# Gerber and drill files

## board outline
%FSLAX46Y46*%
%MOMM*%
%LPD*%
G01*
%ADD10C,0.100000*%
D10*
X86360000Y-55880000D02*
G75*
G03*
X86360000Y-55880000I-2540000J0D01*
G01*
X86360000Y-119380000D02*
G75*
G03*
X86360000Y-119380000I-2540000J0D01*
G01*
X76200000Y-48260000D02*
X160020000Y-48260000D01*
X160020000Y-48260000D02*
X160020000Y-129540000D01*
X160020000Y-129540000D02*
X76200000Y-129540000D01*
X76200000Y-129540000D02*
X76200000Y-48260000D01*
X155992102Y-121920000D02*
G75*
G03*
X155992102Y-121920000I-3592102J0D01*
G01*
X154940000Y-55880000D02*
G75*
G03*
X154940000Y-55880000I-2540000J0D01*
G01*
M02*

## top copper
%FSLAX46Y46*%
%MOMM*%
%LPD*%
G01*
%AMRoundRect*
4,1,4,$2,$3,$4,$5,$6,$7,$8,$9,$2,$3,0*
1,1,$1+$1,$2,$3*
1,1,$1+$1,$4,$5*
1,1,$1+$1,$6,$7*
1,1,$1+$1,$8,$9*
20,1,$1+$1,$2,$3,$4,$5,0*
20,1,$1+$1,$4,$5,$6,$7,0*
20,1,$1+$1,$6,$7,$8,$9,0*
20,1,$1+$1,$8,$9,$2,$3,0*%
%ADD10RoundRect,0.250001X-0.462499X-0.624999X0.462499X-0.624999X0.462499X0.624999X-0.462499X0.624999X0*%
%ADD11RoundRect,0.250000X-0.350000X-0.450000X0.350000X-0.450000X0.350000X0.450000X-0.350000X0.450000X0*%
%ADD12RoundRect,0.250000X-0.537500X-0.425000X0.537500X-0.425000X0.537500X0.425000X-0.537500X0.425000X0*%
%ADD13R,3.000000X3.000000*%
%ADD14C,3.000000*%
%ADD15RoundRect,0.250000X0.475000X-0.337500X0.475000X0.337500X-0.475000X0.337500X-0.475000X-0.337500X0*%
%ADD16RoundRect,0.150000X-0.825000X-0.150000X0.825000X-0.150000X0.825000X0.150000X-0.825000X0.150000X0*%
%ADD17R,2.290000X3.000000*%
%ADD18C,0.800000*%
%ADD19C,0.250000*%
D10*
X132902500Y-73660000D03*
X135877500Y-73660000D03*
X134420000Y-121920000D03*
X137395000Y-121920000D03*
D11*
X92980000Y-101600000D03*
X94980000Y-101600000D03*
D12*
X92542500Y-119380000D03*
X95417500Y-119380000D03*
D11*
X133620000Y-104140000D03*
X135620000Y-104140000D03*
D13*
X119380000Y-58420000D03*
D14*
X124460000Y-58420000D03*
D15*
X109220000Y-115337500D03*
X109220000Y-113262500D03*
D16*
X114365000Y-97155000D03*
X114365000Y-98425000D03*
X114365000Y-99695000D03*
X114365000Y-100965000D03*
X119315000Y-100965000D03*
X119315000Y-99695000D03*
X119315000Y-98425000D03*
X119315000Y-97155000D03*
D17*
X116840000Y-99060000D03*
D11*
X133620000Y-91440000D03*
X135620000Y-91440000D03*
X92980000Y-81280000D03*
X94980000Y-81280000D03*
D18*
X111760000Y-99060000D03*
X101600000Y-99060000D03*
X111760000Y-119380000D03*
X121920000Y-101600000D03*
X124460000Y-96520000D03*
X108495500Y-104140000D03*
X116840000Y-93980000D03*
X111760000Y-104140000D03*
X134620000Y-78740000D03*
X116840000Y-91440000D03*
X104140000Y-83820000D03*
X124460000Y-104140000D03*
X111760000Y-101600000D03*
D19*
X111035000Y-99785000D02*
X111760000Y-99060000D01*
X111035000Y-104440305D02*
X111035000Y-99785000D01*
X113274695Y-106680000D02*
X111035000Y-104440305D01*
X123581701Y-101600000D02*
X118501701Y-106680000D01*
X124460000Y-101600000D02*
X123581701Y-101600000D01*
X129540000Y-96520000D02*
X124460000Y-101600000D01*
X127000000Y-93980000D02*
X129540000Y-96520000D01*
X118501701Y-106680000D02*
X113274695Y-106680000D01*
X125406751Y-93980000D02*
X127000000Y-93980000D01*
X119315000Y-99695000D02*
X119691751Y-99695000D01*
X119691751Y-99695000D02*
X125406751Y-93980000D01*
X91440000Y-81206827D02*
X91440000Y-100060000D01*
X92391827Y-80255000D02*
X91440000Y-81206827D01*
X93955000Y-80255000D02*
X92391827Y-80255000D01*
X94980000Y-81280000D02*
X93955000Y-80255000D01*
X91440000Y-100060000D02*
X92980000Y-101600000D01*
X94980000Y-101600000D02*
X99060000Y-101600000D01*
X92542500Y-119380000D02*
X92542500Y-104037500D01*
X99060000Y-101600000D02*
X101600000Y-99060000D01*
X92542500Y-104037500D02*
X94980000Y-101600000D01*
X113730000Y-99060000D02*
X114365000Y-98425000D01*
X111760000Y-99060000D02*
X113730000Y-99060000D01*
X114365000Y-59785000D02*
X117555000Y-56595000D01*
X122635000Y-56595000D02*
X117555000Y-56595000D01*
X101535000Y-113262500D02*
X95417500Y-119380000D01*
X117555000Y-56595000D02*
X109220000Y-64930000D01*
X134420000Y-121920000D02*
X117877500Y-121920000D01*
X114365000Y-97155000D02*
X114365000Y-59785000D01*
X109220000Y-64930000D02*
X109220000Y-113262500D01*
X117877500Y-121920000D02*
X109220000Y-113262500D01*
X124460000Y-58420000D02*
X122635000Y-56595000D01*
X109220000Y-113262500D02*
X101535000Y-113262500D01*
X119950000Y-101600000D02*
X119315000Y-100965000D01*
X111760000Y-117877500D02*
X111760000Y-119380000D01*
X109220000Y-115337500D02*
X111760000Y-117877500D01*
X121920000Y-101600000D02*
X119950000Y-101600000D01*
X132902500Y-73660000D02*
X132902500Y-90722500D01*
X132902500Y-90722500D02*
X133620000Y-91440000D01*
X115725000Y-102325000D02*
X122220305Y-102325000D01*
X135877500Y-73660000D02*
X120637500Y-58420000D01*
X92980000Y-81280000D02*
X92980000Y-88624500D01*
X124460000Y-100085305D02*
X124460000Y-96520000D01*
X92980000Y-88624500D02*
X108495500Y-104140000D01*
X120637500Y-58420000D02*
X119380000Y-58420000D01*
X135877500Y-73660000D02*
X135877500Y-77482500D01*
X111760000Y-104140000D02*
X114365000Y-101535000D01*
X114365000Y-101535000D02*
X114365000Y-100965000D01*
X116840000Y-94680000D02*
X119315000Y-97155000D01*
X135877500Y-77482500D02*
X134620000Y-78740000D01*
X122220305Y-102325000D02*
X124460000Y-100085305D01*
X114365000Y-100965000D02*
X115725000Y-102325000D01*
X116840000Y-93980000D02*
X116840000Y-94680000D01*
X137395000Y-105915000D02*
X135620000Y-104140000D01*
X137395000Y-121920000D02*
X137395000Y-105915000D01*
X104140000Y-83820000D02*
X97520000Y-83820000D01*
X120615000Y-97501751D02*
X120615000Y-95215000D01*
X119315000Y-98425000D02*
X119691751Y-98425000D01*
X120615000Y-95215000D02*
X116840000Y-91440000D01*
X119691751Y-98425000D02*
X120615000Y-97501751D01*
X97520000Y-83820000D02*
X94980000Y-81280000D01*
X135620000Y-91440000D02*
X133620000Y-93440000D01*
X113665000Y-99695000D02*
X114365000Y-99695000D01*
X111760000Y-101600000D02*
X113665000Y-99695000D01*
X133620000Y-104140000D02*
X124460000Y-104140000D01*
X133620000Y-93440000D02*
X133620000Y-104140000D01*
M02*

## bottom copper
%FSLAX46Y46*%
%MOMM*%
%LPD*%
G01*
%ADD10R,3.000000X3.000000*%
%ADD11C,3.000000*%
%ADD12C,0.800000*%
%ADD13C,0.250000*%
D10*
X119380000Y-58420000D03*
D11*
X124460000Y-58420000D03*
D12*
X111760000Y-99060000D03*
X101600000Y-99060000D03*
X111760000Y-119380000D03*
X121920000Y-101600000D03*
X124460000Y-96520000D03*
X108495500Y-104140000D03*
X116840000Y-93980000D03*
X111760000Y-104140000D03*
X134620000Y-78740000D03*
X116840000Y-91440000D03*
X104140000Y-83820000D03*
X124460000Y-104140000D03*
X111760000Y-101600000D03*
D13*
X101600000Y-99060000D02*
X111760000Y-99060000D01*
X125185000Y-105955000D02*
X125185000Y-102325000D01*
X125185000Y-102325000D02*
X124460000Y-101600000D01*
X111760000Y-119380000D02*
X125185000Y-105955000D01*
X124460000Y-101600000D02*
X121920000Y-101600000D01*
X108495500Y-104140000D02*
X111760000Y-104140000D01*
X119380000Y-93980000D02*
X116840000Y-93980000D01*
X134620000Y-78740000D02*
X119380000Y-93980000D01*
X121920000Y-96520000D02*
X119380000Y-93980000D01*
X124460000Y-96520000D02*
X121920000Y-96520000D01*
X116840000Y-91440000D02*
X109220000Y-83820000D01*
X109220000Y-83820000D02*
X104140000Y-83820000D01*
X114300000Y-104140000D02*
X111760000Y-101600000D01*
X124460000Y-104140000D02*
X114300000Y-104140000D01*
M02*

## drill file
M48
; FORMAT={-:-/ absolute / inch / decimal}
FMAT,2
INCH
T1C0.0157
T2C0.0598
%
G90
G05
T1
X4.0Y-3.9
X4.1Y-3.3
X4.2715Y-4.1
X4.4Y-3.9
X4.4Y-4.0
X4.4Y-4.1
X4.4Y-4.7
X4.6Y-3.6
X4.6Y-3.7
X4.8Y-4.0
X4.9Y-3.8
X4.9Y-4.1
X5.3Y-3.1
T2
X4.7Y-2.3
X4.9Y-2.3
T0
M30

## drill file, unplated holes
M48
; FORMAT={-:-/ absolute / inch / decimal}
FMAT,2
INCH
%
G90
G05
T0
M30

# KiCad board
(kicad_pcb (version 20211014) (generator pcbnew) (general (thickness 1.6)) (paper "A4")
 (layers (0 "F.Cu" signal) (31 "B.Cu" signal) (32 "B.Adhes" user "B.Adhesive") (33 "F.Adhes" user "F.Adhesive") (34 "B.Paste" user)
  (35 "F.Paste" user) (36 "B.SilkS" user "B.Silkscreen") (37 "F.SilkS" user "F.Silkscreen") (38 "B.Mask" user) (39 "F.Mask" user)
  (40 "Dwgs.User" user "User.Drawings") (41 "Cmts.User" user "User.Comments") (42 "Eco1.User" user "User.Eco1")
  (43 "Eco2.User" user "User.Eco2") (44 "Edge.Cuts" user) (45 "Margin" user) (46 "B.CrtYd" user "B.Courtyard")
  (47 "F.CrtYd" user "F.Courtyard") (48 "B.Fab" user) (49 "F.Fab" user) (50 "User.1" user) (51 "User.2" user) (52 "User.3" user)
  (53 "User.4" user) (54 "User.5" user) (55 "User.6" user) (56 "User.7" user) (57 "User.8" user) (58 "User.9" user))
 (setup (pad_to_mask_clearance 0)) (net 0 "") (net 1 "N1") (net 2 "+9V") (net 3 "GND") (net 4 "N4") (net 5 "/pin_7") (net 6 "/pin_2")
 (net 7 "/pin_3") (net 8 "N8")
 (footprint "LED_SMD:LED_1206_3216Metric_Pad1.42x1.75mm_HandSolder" (layer "F.Cu") (at 134.39 73.66)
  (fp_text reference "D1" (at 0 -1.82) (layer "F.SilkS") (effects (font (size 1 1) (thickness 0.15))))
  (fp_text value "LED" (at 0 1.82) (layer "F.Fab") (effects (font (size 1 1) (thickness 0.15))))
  (pad "1" smd roundrect (at -1.4875 0) (size 1.425 1.75) (layers "F.Cu" "F.Paste" "F.Mask") (roundrect_rratio 0.1754392982) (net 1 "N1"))
  (pad "2" smd roundrect (at 1.4875 0) (size 1.425 1.75) (layers "F.Cu" "F.Paste" "F.Mask") (roundrect_rratio 0.1754392982) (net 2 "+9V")))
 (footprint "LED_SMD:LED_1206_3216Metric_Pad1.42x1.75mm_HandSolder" (layer "F.Cu") (at 135.9075 121.92)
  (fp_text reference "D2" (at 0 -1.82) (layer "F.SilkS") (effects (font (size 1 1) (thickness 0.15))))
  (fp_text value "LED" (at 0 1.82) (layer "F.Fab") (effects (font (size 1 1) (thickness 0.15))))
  (pad "1" smd roundrect (at -1.4875 0) (size 1.425 1.75) (layers "F.Cu" "F.Paste" "F.Mask") (roundrect_rratio 0.1754392982) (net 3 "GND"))
  (pad "2" smd roundrect (at 1.4875 0) (size 1.425 1.75) (layers "F.Cu" "F.Paste" "F.Mask") (roundrect_rratio 0.1754392982) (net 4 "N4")))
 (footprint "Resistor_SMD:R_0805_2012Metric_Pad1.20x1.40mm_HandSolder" (layer "F.Cu") (at 93.98 101.6)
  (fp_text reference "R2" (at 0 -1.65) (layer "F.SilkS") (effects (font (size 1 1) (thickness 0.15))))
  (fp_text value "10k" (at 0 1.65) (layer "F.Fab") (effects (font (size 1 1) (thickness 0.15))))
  (pad "1" smd roundrect (at -1 0) (size 1.2 1.4) (layers "F.Cu" "F.Paste" "F.Mask") (roundrect_rratio 0.2083333333) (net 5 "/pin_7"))
  (pad "2" smd roundrect (at 1 0) (size 1.2 1.4) (layers "F.Cu" "F.Paste" "F.Mask") (roundrect_rratio 0.2083333333) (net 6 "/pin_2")))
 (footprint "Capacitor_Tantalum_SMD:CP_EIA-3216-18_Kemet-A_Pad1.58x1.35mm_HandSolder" (layer "F.Cu") (at 93.98 119.38)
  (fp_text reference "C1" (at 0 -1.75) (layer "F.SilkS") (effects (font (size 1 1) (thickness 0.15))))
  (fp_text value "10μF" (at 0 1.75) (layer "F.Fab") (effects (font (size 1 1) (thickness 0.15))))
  (pad "1" smd roundrect (at -1.4375 0) (size 1.575 1.35) (layers "F.Cu" "F.Paste" "F.Mask") (roundrect_rratio 0.1851851852)
   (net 6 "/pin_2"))
  (pad "2" smd roundrect (at 1.4375 0) (size 1.575 1.35) (layers "F.Cu" "F.Paste" "F.Mask") (roundrect_rratio 0.1851851852) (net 3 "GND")))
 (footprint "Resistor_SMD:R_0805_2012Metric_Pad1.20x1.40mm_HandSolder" (layer "F.Cu") (at 134.62 104.14)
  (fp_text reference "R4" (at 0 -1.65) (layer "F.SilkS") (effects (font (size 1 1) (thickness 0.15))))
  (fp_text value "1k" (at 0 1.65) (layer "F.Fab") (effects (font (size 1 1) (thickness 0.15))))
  (pad "1" smd roundrect (at -1 0) (size 1.2 1.4) (layers "F.Cu" "F.Paste" "F.Mask") (roundrect_rratio 0.2083333333) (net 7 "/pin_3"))
  (pad "2" smd roundrect (at 1 0) (size 1.2 1.4) (layers "F.Cu" "F.Paste" "F.Mask") (roundrect_rratio 0.2083333333) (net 4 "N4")))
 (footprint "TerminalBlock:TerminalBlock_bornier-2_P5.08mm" (layer "F.Cu") (at 119.38 58.42)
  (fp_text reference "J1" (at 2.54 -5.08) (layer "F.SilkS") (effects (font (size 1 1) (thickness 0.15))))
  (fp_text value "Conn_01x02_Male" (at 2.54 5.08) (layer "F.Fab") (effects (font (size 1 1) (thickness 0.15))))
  (pad "1" thru_hole rect (at 0 0) (size 3 3) (drill 1.52) (layers *.Cu *.Mask) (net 2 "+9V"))
  (pad "2" thru_hole circle (at 5.08 0) (size 3 3) (drill 1.52) (layers *.Cu *.Mask) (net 3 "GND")))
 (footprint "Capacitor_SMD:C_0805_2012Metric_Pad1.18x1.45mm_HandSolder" (layer "F.Cu") (at 109.22 114.3 90)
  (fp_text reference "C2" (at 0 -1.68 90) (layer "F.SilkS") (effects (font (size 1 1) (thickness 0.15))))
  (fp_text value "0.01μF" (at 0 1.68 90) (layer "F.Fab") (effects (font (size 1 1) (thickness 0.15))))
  (pad "1" smd roundrect (at -1.0375 0 90) (size 1.175 1.45) (layers "F.Cu" "F.Paste" "F.Mask") (roundrect_rratio 0.2127659574) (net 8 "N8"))
  (pad "2" smd roundrect (at 1.0375 0 90) (size 1.175 1.45) (layers "F.Cu" "F.Paste" "F.Mask") (roundrect_rratio 0.2127659574) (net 3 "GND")))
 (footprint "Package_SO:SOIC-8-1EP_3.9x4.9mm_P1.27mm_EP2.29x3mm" (layer "F.Cu") (at 116.84 99.06)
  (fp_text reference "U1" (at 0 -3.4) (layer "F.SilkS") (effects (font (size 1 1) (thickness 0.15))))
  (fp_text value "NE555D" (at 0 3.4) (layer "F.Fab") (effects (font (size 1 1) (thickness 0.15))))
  (pad "" smd roundrect (at 0.57 0.75) (size 0.92 1.21) (layers "F.Paste") (roundrect_rratio 0.25))
  (pad "" smd roundrect (at 0.57 -0.75) (size 0.92 1.21) (layers "F.Paste") (roundrect_rratio 0.25))
  (pad "" smd roundrect (at -0.57 0.75) (size 0.92 1.21) (layers "F.Paste") (roundrect_rratio 0.25))
  (pad "" smd roundrect (at -0.57 -0.75) (size 0.92 1.21) (layers "F.Paste") (roundrect_rratio 0.25))
  (pad "1" smd roundrect (at -2.475 -1.905) (size 1.95 0.6) (layers "F.Cu" "F.Paste" "F.Mask") (roundrect_rratio 0.25) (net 3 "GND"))
  (pad "2" smd roundrect (at -2.475 -0.635) (size 1.95 0.6) (layers "F.Cu" "F.Paste" "F.Mask") (roundrect_rratio 0.25) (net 6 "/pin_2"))
  (pad "3" smd roundrect (at -2.475 0.635) (size 1.95 0.6) (layers "F.Cu" "F.Paste" "F.Mask") (roundrect_rratio 0.25) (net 7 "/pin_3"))
  (pad "4" smd roundrect (at -2.475 1.905) (size 1.95 0.6) (layers "F.Cu" "F.Paste" "F.Mask") (roundrect_rratio 0.25) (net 2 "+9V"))
  (pad "5" smd roundrect (at 2.475 1.905) (size 1.95 0.6) (layers "F.Cu" "F.Paste" "F.Mask") (roundrect_rratio 0.25) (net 8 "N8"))
  (pad "6" smd roundrect (at 2.475 0.635) (size 1.95 0.6) (layers "F.Cu" "F.Paste" "F.Mask") (roundrect_rratio 0.25) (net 6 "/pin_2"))
  (pad "7" smd roundrect (at 2.475 -0.635) (size 1.95 0.6) (layers "F.Cu" "F.Paste" "F.Mask") (roundrect_rratio 0.25) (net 5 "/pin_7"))
  (pad "8" smd roundrect (at 2.475 -1.905) (size 1.95 0.6) (layers "F.Cu" "F.Paste" "F.Mask") (roundrect_rratio 0.25) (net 2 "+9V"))
  (pad "9" smd rect (at 0 0) (size 2.29 3) (layers "F.Cu" "F.Mask")))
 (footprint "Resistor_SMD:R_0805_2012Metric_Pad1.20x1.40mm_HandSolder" (layer "F.Cu") (at 134.62 91.44)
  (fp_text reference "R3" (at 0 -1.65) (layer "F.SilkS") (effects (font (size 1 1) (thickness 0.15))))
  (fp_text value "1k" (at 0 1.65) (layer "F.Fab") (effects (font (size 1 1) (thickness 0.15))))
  (pad "1" smd roundrect (at -1 0) (size 1.2 1.4) (layers "F.Cu" "F.Paste" "F.Mask") (roundrect_rratio 0.2083333333) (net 1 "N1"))
  (pad "2" smd roundrect (at 1 0) (size 1.2 1.4) (layers "F.Cu" "F.Paste" "F.Mask") (roundrect_rratio 0.2083333333) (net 7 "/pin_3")))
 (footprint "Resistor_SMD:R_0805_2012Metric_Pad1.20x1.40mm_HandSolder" (layer "F.Cu") (at 93.98 81.28)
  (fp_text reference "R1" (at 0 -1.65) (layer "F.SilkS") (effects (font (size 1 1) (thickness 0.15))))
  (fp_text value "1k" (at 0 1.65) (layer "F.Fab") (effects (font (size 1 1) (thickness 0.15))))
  (pad "1" smd roundrect (at -1 0) (size 1.2 1.4) (layers "F.Cu" "F.Paste" "F.Mask") (roundrect_rratio 0.2083333333) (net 2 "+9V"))
  (pad "2" smd roundrect (at 1 0) (size 1.2 1.4) (layers "F.Cu" "F.Paste" "F.Mask") (roundrect_rratio 0.2083333333) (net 5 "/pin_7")))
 (gr_circle (center 83.82 55.88) (end 83.82 53.34) (layer "Edge.Cuts") (width 0.1) (fill none))
 (gr_circle (center 83.82 119.38) (end 83.82 116.84) (layer "Edge.Cuts") (width 0.1) (fill none))
 (gr_rect (start 76.2 48.26) (end 160.02 129.54) (layer "Edge.Cuts") (width 0.1) (fill none))
 (gr_circle (center 152.4 121.92) (end 154.94 124.46) (layer "Edge.Cuts") (width 0.1) (fill none))
 (gr_circle (center 152.4 55.88) (end 152.4 58.42) (layer "Edge.Cuts") (width 0.1) (fill none))
 (segment (start 94.98 101.6) (end 99.06 101.6) (width 0.25) (layer "F.Cu") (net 6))
 (segment (start 92.5425 119.38) (end 92.5425 104.0375) (width 0.25) (layer "F.Cu") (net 6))
 (segment (start 111.035 104.440305) (end 111.035 99.785) (width 0.25) (layer "F.Cu") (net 6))
 (segment (start 99.06 101.6) (end 101.6 99.06) (width 0.25) (layer "F.Cu") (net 6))
 (segment (start 113.274695 106.68) (end 111.035 104.440305) (width 0.25) (layer "F.Cu") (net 6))
 (segment (start 123.581701 101.6) (end 118.501701 106.68) (width 0.25) (layer "F.Cu") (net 6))
 (segment (start 111.035 99.785) (end 111.76 99.06) (width 0.25) (layer "F.Cu") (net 6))
 (segment (start 92.5425 104.0375) (end 94.98 101.6) (width 0.25) (layer "F.Cu") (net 6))
 (segment (start 113.73 99.06) (end 114.365 98.425) (width 0.25) (layer "F.Cu") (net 6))
 (segment (start 124.46 101.6) (end 123.581701 101.6) (width 0.25) (layer "F.Cu") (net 6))
 (segment (start 129.54 96.52) (end 124.46 101.6) (width 0.25) (layer "F.Cu") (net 6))
 (segment (start 127 93.98) (end 129.54 96.52) (width 0.25) (layer "F.Cu") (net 6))
 (segment (start 119.691751 99.695) (end 125.406751 93.98) (width 0.25) (layer "F.Cu") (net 6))
 (segment (start 119.315 99.695) (end 119.691751 99.695) (width 0.25) (layer "F.Cu") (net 6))
 (segment (start 125.406751 93.98) (end 127 93.98) (width 0.25) (layer "F.Cu") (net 6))
 (segment (start 118.501701 106.68) (end 113.274695 106.68) (width 0.25) (layer "F.Cu") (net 6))
 (segment (start 111.76 99.06) (end 113.73 99.06) (width 0.25) (layer "F.Cu") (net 6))
 (via (at 111.76 99.06) (size 0.8) (drill 0.4) (layers "F.Cu" "B.Cu") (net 6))
 (via (at 101.6 99.06) (size 0.8) (drill 0.4) (layers "F.Cu" "B.Cu") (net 6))
 (segment (start 101.6 99.06) (end 111.76 99.06) (width 0.25) (layer "B.Cu") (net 6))
 (segment (start 114.365 59.785) (end 117.555 56.595) (width 0.25) (layer "F.Cu") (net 3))
 (segment (start 122.635 56.595) (end 117.555 56.595) (width 0.25) (layer "F.Cu") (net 3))
 (segment (start 101.535 113.2625) (end 95.4175 119.38) (width 0.25) (layer "F.Cu") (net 3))
 (segment (start 117.555 56.595) (end 109.22 64.93) (width 0.25) (layer "F.Cu") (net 3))
 (segment (start 134.42 121.92) (end 117.8775 121.92) (width 0.25) (layer "F.Cu") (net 3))
 (segment (start 114.365 97.155) (end 114.365 59.785) (width 0.25) (layer "F.Cu") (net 3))
 (segment (start 109.22 64.93) (end 109.22 113.2625) (width 0.25) (layer "F.Cu") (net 3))
 (segment (start 117.8775 121.92) (end 109.22 113.2625) (width 0.25) (layer "F.Cu") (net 3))
 (segment (start 124.46 58.42) (end 122.635 56.595) (width 0.25) (layer "F.Cu") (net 3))
 (segment (start 109.22 113.2625) (end 101.535 113.2625) (width 0.25) (layer "F.Cu") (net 3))
 (segment (start 119.95 101.6) (end 119.315 100.965) (width 0.25) (layer "F.Cu") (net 8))
 (segment (start 111.76 117.8775) (end 111.76 119.38) (width 0.25) (layer "F.Cu") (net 8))
 (segment (start 109.22 115.3375) (end 111.76 117.8775) (width 0.25) (layer "F.Cu") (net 8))
 (segment (start 121.92 101.6) (end 119.95 101.6) (width 0.25) (layer "F.Cu") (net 8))
 (via (at 111.76 119.38) (size 0.8) (drill 0.4) (layers "F.Cu" "B.Cu") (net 8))
 (via (at 121.92 101.6) (size 0.8) (drill 0.4) (layers "F.Cu" "B.Cu") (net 8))
 (segment (start 125.185 105.955) (end 125.185 102.325) (width 0.25) (layer "B.Cu") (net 8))
 (segment (start 125.185 102.325) (end 124.46 101.6) (width 0.25) (layer "B.Cu") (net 8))
 (segment (start 111.76 119.38) (end 125.185 105.955) (width 0.25) (layer "B.Cu") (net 8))
 (segment (start 124.46 101.6) (end 121.92 101.6) (width 0.25) (layer "B.Cu") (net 8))
 (segment (start 132.9025 73.66) (end 132.9025 90.7225) (width 0.25) (layer "F.Cu") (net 1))
 (segment (start 132.9025 90.7225) (end 133.62 91.44) (width 0.25) (layer "F.Cu") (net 1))
 (segment (start 115.725 102.325) (end 122.220305 102.325) (width 0.25) (layer "F.Cu") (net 2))
 (segment (start 135.8775 73.66) (end 120.6375 58.42) (width 0.25) (layer "F.Cu") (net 2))
 (segment (start 92.98 81.28) (end 92.98 88.6245) (width 0.25) (layer "F.Cu") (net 2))
 (segment (start 124.46 100.085305) (end 124.46 96.52) (width 0.25) (layer "F.Cu") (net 2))
 (segment (start 92.98 88.6245) (end 108.4955 104.14) (width 0.25) (layer "F.Cu") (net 2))
 (segment (start 120.6375 58.42) (end 119.38 58.42) (width 0.25) (layer "F.Cu") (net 2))
 (segment (start 135.8775 73.66) (end 135.8775 77.4825) (width 0.25) (layer "F.Cu") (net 2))
 (segment (start 111.76 104.14) (end 114.365 101.535) (width 0.25) (layer "F.Cu") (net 2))
 (segment (start 114.365 101.535) (end 114.365 100.965) (width 0.25) (layer "F.Cu") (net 2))
 (segment (start 116.84 94.68) (end 119.315 97.155) (width 0.25) (layer "F.Cu") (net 2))
 (segment (start 135.8775 77.4825) (end 134.62 78.74) (width 0.25) (layer "F.Cu") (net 2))
 (segment (start 122.220305 102.325) (end 124.46 100.085305) (width 0.25) (layer "F.Cu") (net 2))
 (segment (start 114.365 100.965) (end 115.725 102.325) (width 0.25) (layer "F.Cu") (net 2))
 (segment (start 116.84 93.98) (end 116.84 94.68) (width 0.25) (layer "F.Cu") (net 2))
 (via (at 124.46 96.52) (size 0.8) (drill 0.4) (layers "F.Cu" "B.Cu") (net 2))
 (via (at 108.4955 104.14) (size 0.8) (drill 0.4) (layers "F.Cu" "B.Cu") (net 2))
 (via (at 116.84 93.98) (size 0.8) (drill 0.4) (layers "F.Cu" "B.Cu") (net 2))
 (via (at 111.76 104.14) (size 0.8) (drill 0.4) (layers "F.Cu" "B.Cu") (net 2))
 (via (at 134.62 78.74) (size 0.8) (drill 0.4) (layers "F.Cu" "B.Cu") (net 2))
 (segment (start 108.4955 104.14) (end 111.76 104.14) (width 0.25) (layer "B.Cu") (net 2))
 (segment (start 119.38 93.98) (end 116.84 93.98) (width 0.25) (layer "B.Cu") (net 2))
 (segment (start 134.62 78.74) (end 119.38 93.98) (width 0.25) (layer "B.Cu") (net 2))
 (segment (start 121.92 96.52) (end 119.38 93.98) (width 0.25) (layer "B.Cu") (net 2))
 (segment (start 124.46 96.52) (end 121.92 96.52) (width 0.25) (layer "B.Cu") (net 2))
 (segment (start 137.395 105.915) (end 135.62 104.14) (width 0.25) (layer "F.Cu") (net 4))
 (segment (start 137.395 121.92) (end 137.395 105.915) (width 0.25) (layer "F.Cu") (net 4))
 (segment (start 104.14 83.82) (end 97.52 83.82) (width 0.25) (layer "F.Cu") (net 5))
 (segment (start 93.955 80.255) (end 92.391827 80.255) (width 0.25) (layer "F.Cu") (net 5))
 (segment (start 92.391827 80.255) (end 91.44 81.206827) (width 0.25) (layer "F.Cu") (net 5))
 (segment (start 91.44 100.06) (end 92.98 101.6) (width 0.25) (layer "F.Cu") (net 5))
 (segment (start 120.615 97.501751) (end 120.615 95.215) (width 0.25) (layer "F.Cu") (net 5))
 (segment (start 94.98 81.28) (end 93.955 80.255) (width 0.25) (layer "F.Cu") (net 5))
 (segment (start 119.315 98.425) (end 119.691751 98.425) (width 0.25) (layer "F.Cu") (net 5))
 (segment (start 120.615 95.215) (end 116.84 91.44) (width 0.25) (layer "F.Cu") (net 5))
 (segment (start 91.44 81.206827) (end 91.44 100.06) (width 0.25) (layer "F.Cu") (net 5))
 (segment (start 119.691751 98.425) (end 120.615 97.501751) (width 0.25) (layer "F.Cu") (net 5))
 (segment (start 97.52 83.82) (end 94.98 81.28) (width 0.25) (layer "F.Cu") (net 5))
 (via (at 116.84 91.44) (size 0.8) (drill 0.4) (layers "F.Cu" "B.Cu") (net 5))
 (via (at 104.14 83.82) (size 0.8) (drill 0.4) (layers "F.Cu" "B.Cu") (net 5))
 (segment (start 116.84 91.44) (end 109.22 83.82) (width 0.25) (layer "B.Cu") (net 5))
 (segment (start 109.22 83.82) (end 104.14 83.82) (width 0.25) (layer "B.Cu") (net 5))
 (segment (start 135.62 91.44) (end 133.62 93.44) (width 0.25) (layer "F.Cu") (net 7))
 (segment (start 113.665 99.695) (end 114.365 99.695) (width 0.25) (layer "F.Cu") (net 7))
 (segment (start 111.76 101.6) (end 113.665 99.695) (width 0.25) (layer "F.Cu") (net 7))
 (segment (start 133.62 104.14) (end 124.46 104.14) (width 0.25) (layer "F.Cu") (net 7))
 (segment (start 133.62 93.44) (end 133.62 104.14) (width 0.25) (layer "F.Cu") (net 7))
 (via (at 124.46 104.14) (size 0.8) (drill 0.4) (layers "F.Cu" "B.Cu") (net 7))
 (via (at 111.76 101.6) (size 0.8) (drill 0.4) (layers "F.Cu" "B.Cu") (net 7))
 (segment (start 114.3 104.14) (end 111.76 101.6) (width 0.25) (layer "B.Cu") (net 7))
 (segment (start 124.46 104.14) (end 114.3 104.14) (width 0.25) (layer "B.Cu") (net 7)))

